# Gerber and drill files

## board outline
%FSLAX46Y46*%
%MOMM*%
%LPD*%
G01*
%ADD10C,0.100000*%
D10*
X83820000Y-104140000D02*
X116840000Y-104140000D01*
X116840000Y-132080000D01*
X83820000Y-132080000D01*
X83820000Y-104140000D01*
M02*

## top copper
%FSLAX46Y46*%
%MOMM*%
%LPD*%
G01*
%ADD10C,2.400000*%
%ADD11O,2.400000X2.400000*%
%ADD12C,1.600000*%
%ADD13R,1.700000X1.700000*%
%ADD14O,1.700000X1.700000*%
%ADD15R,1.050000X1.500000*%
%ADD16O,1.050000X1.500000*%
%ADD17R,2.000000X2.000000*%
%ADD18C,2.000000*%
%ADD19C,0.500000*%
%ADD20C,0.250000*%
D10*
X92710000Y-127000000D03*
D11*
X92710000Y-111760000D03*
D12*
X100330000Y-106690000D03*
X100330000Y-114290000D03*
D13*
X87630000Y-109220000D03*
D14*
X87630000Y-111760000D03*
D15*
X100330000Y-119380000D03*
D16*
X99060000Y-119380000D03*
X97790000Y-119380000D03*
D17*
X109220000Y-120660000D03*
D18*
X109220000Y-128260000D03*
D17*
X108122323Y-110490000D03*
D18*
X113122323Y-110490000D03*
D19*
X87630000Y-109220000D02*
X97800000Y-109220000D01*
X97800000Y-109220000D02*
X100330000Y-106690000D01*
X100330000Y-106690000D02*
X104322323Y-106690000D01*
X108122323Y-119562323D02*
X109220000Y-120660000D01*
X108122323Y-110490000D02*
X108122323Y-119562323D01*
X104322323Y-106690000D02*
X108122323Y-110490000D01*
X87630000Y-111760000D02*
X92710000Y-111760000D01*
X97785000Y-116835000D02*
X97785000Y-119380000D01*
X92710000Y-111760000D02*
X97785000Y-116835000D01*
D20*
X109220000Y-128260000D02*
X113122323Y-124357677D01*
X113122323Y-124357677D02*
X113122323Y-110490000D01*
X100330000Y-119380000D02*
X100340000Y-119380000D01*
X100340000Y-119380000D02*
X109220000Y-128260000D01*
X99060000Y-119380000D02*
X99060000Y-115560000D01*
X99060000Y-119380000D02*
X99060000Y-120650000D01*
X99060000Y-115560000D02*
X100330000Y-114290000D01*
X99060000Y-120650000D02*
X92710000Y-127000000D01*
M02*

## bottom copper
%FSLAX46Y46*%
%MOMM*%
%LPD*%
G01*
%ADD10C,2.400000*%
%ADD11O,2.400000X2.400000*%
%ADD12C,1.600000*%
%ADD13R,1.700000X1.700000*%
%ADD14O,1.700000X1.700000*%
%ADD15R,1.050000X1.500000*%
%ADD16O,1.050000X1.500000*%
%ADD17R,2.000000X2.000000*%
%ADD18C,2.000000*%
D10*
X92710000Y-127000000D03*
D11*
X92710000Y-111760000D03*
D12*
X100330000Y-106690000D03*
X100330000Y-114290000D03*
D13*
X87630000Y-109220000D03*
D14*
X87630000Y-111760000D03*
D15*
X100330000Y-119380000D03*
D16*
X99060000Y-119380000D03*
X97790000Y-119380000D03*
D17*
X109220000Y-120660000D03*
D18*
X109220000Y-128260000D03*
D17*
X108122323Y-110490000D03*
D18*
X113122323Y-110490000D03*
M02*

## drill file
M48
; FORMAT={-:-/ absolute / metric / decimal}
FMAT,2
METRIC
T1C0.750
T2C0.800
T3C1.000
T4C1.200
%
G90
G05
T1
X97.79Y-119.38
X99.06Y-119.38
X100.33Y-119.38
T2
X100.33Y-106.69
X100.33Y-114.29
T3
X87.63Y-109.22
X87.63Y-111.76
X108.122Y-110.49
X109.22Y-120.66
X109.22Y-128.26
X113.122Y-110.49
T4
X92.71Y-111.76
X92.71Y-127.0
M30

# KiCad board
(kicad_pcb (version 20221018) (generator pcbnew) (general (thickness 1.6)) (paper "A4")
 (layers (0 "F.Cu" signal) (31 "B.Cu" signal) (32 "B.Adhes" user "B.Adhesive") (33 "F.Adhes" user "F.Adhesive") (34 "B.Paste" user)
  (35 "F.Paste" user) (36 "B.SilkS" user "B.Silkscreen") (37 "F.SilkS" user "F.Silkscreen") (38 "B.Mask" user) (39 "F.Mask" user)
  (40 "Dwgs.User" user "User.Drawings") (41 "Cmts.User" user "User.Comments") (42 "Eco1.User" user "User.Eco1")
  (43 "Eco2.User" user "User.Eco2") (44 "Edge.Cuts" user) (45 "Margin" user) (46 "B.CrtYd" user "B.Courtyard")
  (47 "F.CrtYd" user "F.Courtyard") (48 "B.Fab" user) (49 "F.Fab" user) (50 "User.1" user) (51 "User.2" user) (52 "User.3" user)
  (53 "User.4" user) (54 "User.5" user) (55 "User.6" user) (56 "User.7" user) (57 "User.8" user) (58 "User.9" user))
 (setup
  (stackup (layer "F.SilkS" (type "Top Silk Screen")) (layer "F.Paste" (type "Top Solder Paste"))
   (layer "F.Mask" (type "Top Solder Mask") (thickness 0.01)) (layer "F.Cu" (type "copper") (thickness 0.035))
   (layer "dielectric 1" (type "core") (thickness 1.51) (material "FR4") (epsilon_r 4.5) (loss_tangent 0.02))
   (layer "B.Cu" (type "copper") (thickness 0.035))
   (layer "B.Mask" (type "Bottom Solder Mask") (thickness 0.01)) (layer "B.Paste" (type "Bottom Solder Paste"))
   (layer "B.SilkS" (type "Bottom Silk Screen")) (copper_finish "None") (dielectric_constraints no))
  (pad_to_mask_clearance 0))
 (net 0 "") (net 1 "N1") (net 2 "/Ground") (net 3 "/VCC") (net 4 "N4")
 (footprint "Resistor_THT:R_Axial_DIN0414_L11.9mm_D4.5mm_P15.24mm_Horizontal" (layer "F.Cu") (at 92.71 127 90)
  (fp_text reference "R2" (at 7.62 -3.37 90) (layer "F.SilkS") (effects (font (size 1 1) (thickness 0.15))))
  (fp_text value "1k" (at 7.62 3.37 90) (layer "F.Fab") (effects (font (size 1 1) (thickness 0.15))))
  (pad "1" thru_hole circle (at 0 0 90) (size 2.4 2.4) (drill 1.2) (layers "*.Cu" "*.Mask") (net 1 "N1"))
  (pad "2" thru_hole oval (at 15.24 0 90) (size 2.4 2.4) (drill 1.2) (layers "*.Cu" "*.Mask") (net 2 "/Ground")))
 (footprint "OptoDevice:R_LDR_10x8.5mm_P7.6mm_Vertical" (layer "F.Cu") (at 100.33 106.69 -90)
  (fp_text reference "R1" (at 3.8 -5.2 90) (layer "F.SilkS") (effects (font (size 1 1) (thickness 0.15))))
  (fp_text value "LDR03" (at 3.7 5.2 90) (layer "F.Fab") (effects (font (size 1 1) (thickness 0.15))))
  (pad "1" thru_hole circle (at 0 0 270) (size 1.6 1.6) (drill 0.8) (layers "*.Cu" "*.Mask") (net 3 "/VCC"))
  (pad "2" thru_hole circle (at 7.6 0 270) (size 1.6 1.6) (drill 0.8) (layers "*.Cu" "*.Mask") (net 1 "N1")))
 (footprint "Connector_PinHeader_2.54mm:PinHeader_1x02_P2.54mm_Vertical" (layer "F.Cu") (at 87.63 109.22)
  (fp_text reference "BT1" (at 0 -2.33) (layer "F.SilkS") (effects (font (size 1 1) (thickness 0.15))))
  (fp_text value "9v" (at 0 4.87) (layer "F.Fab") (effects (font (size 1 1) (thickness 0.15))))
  (pad "1" thru_hole rect (at 0 0) (size 1.7 1.7) (drill 1) (layers "*.Cu" "*.Mask") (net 3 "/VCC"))
  (pad "2" thru_hole oval (at 0 2.54) (size 1.7 1.7) (drill 1) (layers "*.Cu" "*.Mask") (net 2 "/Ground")))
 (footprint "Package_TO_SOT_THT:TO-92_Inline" (layer "F.Cu") (at 100.33 119.38 180)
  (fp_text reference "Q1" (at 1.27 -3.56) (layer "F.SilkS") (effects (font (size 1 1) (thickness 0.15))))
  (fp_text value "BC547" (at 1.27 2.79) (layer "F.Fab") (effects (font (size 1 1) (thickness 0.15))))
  (pad "1" thru_hole rect (at 0 0 180) (size 1.05 1.5) (drill 0.75) (layers "*.Cu" "*.Mask") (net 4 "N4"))
  (pad "2" thru_hole oval (at 1.27 0 180) (size 1.05 1.5) (drill 0.75) (layers "*.Cu" "*.Mask") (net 1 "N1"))
  (pad "3" thru_hole oval (at 2.54 0 180) (size 1.05 1.5) (drill 0.75) (layers "*.Cu" "*.Mask") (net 2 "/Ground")))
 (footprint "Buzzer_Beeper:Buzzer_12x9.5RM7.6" (layer "F.Cu") (at 109.22 120.66 -90)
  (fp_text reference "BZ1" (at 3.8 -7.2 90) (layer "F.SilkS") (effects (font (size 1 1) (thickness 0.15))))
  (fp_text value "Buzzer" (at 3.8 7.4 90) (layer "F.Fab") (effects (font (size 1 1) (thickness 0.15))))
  (pad "1" thru_hole rect (at 0 0 270) (size 2 2) (drill 1) (layers "*.Cu" "*.Mask") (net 3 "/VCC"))
  (pad "2" thru_hole circle (at 7.6 0 270) (size 2 2) (drill 1) (layers "*.Cu" "*.Mask") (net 4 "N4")))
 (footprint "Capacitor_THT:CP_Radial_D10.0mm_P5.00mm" (layer "F.Cu") (at 108.122323 110.49)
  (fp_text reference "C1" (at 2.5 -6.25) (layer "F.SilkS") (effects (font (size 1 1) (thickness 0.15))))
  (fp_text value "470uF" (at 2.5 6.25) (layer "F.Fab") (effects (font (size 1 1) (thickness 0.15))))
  (pad "1" thru_hole rect (at 0 0) (size 2 2) (drill 1) (layers "*.Cu" "*.Mask") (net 3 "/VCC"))
  (pad "2" thru_hole circle (at 5 0) (size 2 2) (drill 1) (layers "*.Cu" "*.Mask") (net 4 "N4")))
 (gr_rect (start 83.82 104.14) (end 116.84 132.08) (stroke (width 0.1) (type default)) (fill none) (layer "Edge.Cuts"))
 (segment (start 87.63 109.22) (end 97.8 109.22) (width 0.5) (layer "F.Cu") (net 3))
 (segment (start 97.8 109.22) (end 100.33 106.69) (width 0.5) (layer "F.Cu") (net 3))
 (segment (start 100.33 106.69) (end 104.322323 106.69) (width 0.5) (layer "F.Cu") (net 3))
 (segment (start 108.122323 119.562323) (end 109.22 120.66) (width 0.5) (layer "F.Cu") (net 3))
 (segment (start 108.122323 110.49) (end 108.122323 119.562323) (width 0.5) (layer "F.Cu") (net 3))
 (segment (start 104.322323 106.69) (end 108.122323 110.49) (width 0.5) (layer "F.Cu") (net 3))
 (segment (start 87.63 111.76) (end 92.71 111.76) (width 0.5) (layer "F.Cu") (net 2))
 (segment (start 97.785 116.835) (end 97.785 119.38) (width 0.5) (layer "F.Cu") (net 2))
 (segment (start 92.71 111.76) (end 97.785 116.835) (width 0.5) (layer "F.Cu") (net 2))
 (segment (start 109.22 128.26) (end 113.122323 124.357677) (width 0.25) (layer "F.Cu") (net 4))
 (segment (start 113.122323 124.357677) (end 113.122323 110.49) (width 0.25) (layer "F.Cu") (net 4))
 (segment (start 100.33 119.38) (end 100.34 119.38) (width 0.25) (layer "F.Cu") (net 4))
 (segment (start 100.34 119.38) (end 109.22 128.26) (width 0.25) (layer "F.Cu") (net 4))
 (segment (start 99.06 119.38) (end 99.06 115.56) (width 0.25) (layer "F.Cu") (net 1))
 (segment (start 99.06 119.38) (end 99.06 120.65) (width 0.25) (layer "F.Cu") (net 1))
 (segment (start 99.06 115.56) (end 100.33 114.29) (width 0.25) (layer "F.Cu") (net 1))
 (segment (start 99.06 120.65) (end 92.71 127) (width 0.25) (layer "F.Cu") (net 1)))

